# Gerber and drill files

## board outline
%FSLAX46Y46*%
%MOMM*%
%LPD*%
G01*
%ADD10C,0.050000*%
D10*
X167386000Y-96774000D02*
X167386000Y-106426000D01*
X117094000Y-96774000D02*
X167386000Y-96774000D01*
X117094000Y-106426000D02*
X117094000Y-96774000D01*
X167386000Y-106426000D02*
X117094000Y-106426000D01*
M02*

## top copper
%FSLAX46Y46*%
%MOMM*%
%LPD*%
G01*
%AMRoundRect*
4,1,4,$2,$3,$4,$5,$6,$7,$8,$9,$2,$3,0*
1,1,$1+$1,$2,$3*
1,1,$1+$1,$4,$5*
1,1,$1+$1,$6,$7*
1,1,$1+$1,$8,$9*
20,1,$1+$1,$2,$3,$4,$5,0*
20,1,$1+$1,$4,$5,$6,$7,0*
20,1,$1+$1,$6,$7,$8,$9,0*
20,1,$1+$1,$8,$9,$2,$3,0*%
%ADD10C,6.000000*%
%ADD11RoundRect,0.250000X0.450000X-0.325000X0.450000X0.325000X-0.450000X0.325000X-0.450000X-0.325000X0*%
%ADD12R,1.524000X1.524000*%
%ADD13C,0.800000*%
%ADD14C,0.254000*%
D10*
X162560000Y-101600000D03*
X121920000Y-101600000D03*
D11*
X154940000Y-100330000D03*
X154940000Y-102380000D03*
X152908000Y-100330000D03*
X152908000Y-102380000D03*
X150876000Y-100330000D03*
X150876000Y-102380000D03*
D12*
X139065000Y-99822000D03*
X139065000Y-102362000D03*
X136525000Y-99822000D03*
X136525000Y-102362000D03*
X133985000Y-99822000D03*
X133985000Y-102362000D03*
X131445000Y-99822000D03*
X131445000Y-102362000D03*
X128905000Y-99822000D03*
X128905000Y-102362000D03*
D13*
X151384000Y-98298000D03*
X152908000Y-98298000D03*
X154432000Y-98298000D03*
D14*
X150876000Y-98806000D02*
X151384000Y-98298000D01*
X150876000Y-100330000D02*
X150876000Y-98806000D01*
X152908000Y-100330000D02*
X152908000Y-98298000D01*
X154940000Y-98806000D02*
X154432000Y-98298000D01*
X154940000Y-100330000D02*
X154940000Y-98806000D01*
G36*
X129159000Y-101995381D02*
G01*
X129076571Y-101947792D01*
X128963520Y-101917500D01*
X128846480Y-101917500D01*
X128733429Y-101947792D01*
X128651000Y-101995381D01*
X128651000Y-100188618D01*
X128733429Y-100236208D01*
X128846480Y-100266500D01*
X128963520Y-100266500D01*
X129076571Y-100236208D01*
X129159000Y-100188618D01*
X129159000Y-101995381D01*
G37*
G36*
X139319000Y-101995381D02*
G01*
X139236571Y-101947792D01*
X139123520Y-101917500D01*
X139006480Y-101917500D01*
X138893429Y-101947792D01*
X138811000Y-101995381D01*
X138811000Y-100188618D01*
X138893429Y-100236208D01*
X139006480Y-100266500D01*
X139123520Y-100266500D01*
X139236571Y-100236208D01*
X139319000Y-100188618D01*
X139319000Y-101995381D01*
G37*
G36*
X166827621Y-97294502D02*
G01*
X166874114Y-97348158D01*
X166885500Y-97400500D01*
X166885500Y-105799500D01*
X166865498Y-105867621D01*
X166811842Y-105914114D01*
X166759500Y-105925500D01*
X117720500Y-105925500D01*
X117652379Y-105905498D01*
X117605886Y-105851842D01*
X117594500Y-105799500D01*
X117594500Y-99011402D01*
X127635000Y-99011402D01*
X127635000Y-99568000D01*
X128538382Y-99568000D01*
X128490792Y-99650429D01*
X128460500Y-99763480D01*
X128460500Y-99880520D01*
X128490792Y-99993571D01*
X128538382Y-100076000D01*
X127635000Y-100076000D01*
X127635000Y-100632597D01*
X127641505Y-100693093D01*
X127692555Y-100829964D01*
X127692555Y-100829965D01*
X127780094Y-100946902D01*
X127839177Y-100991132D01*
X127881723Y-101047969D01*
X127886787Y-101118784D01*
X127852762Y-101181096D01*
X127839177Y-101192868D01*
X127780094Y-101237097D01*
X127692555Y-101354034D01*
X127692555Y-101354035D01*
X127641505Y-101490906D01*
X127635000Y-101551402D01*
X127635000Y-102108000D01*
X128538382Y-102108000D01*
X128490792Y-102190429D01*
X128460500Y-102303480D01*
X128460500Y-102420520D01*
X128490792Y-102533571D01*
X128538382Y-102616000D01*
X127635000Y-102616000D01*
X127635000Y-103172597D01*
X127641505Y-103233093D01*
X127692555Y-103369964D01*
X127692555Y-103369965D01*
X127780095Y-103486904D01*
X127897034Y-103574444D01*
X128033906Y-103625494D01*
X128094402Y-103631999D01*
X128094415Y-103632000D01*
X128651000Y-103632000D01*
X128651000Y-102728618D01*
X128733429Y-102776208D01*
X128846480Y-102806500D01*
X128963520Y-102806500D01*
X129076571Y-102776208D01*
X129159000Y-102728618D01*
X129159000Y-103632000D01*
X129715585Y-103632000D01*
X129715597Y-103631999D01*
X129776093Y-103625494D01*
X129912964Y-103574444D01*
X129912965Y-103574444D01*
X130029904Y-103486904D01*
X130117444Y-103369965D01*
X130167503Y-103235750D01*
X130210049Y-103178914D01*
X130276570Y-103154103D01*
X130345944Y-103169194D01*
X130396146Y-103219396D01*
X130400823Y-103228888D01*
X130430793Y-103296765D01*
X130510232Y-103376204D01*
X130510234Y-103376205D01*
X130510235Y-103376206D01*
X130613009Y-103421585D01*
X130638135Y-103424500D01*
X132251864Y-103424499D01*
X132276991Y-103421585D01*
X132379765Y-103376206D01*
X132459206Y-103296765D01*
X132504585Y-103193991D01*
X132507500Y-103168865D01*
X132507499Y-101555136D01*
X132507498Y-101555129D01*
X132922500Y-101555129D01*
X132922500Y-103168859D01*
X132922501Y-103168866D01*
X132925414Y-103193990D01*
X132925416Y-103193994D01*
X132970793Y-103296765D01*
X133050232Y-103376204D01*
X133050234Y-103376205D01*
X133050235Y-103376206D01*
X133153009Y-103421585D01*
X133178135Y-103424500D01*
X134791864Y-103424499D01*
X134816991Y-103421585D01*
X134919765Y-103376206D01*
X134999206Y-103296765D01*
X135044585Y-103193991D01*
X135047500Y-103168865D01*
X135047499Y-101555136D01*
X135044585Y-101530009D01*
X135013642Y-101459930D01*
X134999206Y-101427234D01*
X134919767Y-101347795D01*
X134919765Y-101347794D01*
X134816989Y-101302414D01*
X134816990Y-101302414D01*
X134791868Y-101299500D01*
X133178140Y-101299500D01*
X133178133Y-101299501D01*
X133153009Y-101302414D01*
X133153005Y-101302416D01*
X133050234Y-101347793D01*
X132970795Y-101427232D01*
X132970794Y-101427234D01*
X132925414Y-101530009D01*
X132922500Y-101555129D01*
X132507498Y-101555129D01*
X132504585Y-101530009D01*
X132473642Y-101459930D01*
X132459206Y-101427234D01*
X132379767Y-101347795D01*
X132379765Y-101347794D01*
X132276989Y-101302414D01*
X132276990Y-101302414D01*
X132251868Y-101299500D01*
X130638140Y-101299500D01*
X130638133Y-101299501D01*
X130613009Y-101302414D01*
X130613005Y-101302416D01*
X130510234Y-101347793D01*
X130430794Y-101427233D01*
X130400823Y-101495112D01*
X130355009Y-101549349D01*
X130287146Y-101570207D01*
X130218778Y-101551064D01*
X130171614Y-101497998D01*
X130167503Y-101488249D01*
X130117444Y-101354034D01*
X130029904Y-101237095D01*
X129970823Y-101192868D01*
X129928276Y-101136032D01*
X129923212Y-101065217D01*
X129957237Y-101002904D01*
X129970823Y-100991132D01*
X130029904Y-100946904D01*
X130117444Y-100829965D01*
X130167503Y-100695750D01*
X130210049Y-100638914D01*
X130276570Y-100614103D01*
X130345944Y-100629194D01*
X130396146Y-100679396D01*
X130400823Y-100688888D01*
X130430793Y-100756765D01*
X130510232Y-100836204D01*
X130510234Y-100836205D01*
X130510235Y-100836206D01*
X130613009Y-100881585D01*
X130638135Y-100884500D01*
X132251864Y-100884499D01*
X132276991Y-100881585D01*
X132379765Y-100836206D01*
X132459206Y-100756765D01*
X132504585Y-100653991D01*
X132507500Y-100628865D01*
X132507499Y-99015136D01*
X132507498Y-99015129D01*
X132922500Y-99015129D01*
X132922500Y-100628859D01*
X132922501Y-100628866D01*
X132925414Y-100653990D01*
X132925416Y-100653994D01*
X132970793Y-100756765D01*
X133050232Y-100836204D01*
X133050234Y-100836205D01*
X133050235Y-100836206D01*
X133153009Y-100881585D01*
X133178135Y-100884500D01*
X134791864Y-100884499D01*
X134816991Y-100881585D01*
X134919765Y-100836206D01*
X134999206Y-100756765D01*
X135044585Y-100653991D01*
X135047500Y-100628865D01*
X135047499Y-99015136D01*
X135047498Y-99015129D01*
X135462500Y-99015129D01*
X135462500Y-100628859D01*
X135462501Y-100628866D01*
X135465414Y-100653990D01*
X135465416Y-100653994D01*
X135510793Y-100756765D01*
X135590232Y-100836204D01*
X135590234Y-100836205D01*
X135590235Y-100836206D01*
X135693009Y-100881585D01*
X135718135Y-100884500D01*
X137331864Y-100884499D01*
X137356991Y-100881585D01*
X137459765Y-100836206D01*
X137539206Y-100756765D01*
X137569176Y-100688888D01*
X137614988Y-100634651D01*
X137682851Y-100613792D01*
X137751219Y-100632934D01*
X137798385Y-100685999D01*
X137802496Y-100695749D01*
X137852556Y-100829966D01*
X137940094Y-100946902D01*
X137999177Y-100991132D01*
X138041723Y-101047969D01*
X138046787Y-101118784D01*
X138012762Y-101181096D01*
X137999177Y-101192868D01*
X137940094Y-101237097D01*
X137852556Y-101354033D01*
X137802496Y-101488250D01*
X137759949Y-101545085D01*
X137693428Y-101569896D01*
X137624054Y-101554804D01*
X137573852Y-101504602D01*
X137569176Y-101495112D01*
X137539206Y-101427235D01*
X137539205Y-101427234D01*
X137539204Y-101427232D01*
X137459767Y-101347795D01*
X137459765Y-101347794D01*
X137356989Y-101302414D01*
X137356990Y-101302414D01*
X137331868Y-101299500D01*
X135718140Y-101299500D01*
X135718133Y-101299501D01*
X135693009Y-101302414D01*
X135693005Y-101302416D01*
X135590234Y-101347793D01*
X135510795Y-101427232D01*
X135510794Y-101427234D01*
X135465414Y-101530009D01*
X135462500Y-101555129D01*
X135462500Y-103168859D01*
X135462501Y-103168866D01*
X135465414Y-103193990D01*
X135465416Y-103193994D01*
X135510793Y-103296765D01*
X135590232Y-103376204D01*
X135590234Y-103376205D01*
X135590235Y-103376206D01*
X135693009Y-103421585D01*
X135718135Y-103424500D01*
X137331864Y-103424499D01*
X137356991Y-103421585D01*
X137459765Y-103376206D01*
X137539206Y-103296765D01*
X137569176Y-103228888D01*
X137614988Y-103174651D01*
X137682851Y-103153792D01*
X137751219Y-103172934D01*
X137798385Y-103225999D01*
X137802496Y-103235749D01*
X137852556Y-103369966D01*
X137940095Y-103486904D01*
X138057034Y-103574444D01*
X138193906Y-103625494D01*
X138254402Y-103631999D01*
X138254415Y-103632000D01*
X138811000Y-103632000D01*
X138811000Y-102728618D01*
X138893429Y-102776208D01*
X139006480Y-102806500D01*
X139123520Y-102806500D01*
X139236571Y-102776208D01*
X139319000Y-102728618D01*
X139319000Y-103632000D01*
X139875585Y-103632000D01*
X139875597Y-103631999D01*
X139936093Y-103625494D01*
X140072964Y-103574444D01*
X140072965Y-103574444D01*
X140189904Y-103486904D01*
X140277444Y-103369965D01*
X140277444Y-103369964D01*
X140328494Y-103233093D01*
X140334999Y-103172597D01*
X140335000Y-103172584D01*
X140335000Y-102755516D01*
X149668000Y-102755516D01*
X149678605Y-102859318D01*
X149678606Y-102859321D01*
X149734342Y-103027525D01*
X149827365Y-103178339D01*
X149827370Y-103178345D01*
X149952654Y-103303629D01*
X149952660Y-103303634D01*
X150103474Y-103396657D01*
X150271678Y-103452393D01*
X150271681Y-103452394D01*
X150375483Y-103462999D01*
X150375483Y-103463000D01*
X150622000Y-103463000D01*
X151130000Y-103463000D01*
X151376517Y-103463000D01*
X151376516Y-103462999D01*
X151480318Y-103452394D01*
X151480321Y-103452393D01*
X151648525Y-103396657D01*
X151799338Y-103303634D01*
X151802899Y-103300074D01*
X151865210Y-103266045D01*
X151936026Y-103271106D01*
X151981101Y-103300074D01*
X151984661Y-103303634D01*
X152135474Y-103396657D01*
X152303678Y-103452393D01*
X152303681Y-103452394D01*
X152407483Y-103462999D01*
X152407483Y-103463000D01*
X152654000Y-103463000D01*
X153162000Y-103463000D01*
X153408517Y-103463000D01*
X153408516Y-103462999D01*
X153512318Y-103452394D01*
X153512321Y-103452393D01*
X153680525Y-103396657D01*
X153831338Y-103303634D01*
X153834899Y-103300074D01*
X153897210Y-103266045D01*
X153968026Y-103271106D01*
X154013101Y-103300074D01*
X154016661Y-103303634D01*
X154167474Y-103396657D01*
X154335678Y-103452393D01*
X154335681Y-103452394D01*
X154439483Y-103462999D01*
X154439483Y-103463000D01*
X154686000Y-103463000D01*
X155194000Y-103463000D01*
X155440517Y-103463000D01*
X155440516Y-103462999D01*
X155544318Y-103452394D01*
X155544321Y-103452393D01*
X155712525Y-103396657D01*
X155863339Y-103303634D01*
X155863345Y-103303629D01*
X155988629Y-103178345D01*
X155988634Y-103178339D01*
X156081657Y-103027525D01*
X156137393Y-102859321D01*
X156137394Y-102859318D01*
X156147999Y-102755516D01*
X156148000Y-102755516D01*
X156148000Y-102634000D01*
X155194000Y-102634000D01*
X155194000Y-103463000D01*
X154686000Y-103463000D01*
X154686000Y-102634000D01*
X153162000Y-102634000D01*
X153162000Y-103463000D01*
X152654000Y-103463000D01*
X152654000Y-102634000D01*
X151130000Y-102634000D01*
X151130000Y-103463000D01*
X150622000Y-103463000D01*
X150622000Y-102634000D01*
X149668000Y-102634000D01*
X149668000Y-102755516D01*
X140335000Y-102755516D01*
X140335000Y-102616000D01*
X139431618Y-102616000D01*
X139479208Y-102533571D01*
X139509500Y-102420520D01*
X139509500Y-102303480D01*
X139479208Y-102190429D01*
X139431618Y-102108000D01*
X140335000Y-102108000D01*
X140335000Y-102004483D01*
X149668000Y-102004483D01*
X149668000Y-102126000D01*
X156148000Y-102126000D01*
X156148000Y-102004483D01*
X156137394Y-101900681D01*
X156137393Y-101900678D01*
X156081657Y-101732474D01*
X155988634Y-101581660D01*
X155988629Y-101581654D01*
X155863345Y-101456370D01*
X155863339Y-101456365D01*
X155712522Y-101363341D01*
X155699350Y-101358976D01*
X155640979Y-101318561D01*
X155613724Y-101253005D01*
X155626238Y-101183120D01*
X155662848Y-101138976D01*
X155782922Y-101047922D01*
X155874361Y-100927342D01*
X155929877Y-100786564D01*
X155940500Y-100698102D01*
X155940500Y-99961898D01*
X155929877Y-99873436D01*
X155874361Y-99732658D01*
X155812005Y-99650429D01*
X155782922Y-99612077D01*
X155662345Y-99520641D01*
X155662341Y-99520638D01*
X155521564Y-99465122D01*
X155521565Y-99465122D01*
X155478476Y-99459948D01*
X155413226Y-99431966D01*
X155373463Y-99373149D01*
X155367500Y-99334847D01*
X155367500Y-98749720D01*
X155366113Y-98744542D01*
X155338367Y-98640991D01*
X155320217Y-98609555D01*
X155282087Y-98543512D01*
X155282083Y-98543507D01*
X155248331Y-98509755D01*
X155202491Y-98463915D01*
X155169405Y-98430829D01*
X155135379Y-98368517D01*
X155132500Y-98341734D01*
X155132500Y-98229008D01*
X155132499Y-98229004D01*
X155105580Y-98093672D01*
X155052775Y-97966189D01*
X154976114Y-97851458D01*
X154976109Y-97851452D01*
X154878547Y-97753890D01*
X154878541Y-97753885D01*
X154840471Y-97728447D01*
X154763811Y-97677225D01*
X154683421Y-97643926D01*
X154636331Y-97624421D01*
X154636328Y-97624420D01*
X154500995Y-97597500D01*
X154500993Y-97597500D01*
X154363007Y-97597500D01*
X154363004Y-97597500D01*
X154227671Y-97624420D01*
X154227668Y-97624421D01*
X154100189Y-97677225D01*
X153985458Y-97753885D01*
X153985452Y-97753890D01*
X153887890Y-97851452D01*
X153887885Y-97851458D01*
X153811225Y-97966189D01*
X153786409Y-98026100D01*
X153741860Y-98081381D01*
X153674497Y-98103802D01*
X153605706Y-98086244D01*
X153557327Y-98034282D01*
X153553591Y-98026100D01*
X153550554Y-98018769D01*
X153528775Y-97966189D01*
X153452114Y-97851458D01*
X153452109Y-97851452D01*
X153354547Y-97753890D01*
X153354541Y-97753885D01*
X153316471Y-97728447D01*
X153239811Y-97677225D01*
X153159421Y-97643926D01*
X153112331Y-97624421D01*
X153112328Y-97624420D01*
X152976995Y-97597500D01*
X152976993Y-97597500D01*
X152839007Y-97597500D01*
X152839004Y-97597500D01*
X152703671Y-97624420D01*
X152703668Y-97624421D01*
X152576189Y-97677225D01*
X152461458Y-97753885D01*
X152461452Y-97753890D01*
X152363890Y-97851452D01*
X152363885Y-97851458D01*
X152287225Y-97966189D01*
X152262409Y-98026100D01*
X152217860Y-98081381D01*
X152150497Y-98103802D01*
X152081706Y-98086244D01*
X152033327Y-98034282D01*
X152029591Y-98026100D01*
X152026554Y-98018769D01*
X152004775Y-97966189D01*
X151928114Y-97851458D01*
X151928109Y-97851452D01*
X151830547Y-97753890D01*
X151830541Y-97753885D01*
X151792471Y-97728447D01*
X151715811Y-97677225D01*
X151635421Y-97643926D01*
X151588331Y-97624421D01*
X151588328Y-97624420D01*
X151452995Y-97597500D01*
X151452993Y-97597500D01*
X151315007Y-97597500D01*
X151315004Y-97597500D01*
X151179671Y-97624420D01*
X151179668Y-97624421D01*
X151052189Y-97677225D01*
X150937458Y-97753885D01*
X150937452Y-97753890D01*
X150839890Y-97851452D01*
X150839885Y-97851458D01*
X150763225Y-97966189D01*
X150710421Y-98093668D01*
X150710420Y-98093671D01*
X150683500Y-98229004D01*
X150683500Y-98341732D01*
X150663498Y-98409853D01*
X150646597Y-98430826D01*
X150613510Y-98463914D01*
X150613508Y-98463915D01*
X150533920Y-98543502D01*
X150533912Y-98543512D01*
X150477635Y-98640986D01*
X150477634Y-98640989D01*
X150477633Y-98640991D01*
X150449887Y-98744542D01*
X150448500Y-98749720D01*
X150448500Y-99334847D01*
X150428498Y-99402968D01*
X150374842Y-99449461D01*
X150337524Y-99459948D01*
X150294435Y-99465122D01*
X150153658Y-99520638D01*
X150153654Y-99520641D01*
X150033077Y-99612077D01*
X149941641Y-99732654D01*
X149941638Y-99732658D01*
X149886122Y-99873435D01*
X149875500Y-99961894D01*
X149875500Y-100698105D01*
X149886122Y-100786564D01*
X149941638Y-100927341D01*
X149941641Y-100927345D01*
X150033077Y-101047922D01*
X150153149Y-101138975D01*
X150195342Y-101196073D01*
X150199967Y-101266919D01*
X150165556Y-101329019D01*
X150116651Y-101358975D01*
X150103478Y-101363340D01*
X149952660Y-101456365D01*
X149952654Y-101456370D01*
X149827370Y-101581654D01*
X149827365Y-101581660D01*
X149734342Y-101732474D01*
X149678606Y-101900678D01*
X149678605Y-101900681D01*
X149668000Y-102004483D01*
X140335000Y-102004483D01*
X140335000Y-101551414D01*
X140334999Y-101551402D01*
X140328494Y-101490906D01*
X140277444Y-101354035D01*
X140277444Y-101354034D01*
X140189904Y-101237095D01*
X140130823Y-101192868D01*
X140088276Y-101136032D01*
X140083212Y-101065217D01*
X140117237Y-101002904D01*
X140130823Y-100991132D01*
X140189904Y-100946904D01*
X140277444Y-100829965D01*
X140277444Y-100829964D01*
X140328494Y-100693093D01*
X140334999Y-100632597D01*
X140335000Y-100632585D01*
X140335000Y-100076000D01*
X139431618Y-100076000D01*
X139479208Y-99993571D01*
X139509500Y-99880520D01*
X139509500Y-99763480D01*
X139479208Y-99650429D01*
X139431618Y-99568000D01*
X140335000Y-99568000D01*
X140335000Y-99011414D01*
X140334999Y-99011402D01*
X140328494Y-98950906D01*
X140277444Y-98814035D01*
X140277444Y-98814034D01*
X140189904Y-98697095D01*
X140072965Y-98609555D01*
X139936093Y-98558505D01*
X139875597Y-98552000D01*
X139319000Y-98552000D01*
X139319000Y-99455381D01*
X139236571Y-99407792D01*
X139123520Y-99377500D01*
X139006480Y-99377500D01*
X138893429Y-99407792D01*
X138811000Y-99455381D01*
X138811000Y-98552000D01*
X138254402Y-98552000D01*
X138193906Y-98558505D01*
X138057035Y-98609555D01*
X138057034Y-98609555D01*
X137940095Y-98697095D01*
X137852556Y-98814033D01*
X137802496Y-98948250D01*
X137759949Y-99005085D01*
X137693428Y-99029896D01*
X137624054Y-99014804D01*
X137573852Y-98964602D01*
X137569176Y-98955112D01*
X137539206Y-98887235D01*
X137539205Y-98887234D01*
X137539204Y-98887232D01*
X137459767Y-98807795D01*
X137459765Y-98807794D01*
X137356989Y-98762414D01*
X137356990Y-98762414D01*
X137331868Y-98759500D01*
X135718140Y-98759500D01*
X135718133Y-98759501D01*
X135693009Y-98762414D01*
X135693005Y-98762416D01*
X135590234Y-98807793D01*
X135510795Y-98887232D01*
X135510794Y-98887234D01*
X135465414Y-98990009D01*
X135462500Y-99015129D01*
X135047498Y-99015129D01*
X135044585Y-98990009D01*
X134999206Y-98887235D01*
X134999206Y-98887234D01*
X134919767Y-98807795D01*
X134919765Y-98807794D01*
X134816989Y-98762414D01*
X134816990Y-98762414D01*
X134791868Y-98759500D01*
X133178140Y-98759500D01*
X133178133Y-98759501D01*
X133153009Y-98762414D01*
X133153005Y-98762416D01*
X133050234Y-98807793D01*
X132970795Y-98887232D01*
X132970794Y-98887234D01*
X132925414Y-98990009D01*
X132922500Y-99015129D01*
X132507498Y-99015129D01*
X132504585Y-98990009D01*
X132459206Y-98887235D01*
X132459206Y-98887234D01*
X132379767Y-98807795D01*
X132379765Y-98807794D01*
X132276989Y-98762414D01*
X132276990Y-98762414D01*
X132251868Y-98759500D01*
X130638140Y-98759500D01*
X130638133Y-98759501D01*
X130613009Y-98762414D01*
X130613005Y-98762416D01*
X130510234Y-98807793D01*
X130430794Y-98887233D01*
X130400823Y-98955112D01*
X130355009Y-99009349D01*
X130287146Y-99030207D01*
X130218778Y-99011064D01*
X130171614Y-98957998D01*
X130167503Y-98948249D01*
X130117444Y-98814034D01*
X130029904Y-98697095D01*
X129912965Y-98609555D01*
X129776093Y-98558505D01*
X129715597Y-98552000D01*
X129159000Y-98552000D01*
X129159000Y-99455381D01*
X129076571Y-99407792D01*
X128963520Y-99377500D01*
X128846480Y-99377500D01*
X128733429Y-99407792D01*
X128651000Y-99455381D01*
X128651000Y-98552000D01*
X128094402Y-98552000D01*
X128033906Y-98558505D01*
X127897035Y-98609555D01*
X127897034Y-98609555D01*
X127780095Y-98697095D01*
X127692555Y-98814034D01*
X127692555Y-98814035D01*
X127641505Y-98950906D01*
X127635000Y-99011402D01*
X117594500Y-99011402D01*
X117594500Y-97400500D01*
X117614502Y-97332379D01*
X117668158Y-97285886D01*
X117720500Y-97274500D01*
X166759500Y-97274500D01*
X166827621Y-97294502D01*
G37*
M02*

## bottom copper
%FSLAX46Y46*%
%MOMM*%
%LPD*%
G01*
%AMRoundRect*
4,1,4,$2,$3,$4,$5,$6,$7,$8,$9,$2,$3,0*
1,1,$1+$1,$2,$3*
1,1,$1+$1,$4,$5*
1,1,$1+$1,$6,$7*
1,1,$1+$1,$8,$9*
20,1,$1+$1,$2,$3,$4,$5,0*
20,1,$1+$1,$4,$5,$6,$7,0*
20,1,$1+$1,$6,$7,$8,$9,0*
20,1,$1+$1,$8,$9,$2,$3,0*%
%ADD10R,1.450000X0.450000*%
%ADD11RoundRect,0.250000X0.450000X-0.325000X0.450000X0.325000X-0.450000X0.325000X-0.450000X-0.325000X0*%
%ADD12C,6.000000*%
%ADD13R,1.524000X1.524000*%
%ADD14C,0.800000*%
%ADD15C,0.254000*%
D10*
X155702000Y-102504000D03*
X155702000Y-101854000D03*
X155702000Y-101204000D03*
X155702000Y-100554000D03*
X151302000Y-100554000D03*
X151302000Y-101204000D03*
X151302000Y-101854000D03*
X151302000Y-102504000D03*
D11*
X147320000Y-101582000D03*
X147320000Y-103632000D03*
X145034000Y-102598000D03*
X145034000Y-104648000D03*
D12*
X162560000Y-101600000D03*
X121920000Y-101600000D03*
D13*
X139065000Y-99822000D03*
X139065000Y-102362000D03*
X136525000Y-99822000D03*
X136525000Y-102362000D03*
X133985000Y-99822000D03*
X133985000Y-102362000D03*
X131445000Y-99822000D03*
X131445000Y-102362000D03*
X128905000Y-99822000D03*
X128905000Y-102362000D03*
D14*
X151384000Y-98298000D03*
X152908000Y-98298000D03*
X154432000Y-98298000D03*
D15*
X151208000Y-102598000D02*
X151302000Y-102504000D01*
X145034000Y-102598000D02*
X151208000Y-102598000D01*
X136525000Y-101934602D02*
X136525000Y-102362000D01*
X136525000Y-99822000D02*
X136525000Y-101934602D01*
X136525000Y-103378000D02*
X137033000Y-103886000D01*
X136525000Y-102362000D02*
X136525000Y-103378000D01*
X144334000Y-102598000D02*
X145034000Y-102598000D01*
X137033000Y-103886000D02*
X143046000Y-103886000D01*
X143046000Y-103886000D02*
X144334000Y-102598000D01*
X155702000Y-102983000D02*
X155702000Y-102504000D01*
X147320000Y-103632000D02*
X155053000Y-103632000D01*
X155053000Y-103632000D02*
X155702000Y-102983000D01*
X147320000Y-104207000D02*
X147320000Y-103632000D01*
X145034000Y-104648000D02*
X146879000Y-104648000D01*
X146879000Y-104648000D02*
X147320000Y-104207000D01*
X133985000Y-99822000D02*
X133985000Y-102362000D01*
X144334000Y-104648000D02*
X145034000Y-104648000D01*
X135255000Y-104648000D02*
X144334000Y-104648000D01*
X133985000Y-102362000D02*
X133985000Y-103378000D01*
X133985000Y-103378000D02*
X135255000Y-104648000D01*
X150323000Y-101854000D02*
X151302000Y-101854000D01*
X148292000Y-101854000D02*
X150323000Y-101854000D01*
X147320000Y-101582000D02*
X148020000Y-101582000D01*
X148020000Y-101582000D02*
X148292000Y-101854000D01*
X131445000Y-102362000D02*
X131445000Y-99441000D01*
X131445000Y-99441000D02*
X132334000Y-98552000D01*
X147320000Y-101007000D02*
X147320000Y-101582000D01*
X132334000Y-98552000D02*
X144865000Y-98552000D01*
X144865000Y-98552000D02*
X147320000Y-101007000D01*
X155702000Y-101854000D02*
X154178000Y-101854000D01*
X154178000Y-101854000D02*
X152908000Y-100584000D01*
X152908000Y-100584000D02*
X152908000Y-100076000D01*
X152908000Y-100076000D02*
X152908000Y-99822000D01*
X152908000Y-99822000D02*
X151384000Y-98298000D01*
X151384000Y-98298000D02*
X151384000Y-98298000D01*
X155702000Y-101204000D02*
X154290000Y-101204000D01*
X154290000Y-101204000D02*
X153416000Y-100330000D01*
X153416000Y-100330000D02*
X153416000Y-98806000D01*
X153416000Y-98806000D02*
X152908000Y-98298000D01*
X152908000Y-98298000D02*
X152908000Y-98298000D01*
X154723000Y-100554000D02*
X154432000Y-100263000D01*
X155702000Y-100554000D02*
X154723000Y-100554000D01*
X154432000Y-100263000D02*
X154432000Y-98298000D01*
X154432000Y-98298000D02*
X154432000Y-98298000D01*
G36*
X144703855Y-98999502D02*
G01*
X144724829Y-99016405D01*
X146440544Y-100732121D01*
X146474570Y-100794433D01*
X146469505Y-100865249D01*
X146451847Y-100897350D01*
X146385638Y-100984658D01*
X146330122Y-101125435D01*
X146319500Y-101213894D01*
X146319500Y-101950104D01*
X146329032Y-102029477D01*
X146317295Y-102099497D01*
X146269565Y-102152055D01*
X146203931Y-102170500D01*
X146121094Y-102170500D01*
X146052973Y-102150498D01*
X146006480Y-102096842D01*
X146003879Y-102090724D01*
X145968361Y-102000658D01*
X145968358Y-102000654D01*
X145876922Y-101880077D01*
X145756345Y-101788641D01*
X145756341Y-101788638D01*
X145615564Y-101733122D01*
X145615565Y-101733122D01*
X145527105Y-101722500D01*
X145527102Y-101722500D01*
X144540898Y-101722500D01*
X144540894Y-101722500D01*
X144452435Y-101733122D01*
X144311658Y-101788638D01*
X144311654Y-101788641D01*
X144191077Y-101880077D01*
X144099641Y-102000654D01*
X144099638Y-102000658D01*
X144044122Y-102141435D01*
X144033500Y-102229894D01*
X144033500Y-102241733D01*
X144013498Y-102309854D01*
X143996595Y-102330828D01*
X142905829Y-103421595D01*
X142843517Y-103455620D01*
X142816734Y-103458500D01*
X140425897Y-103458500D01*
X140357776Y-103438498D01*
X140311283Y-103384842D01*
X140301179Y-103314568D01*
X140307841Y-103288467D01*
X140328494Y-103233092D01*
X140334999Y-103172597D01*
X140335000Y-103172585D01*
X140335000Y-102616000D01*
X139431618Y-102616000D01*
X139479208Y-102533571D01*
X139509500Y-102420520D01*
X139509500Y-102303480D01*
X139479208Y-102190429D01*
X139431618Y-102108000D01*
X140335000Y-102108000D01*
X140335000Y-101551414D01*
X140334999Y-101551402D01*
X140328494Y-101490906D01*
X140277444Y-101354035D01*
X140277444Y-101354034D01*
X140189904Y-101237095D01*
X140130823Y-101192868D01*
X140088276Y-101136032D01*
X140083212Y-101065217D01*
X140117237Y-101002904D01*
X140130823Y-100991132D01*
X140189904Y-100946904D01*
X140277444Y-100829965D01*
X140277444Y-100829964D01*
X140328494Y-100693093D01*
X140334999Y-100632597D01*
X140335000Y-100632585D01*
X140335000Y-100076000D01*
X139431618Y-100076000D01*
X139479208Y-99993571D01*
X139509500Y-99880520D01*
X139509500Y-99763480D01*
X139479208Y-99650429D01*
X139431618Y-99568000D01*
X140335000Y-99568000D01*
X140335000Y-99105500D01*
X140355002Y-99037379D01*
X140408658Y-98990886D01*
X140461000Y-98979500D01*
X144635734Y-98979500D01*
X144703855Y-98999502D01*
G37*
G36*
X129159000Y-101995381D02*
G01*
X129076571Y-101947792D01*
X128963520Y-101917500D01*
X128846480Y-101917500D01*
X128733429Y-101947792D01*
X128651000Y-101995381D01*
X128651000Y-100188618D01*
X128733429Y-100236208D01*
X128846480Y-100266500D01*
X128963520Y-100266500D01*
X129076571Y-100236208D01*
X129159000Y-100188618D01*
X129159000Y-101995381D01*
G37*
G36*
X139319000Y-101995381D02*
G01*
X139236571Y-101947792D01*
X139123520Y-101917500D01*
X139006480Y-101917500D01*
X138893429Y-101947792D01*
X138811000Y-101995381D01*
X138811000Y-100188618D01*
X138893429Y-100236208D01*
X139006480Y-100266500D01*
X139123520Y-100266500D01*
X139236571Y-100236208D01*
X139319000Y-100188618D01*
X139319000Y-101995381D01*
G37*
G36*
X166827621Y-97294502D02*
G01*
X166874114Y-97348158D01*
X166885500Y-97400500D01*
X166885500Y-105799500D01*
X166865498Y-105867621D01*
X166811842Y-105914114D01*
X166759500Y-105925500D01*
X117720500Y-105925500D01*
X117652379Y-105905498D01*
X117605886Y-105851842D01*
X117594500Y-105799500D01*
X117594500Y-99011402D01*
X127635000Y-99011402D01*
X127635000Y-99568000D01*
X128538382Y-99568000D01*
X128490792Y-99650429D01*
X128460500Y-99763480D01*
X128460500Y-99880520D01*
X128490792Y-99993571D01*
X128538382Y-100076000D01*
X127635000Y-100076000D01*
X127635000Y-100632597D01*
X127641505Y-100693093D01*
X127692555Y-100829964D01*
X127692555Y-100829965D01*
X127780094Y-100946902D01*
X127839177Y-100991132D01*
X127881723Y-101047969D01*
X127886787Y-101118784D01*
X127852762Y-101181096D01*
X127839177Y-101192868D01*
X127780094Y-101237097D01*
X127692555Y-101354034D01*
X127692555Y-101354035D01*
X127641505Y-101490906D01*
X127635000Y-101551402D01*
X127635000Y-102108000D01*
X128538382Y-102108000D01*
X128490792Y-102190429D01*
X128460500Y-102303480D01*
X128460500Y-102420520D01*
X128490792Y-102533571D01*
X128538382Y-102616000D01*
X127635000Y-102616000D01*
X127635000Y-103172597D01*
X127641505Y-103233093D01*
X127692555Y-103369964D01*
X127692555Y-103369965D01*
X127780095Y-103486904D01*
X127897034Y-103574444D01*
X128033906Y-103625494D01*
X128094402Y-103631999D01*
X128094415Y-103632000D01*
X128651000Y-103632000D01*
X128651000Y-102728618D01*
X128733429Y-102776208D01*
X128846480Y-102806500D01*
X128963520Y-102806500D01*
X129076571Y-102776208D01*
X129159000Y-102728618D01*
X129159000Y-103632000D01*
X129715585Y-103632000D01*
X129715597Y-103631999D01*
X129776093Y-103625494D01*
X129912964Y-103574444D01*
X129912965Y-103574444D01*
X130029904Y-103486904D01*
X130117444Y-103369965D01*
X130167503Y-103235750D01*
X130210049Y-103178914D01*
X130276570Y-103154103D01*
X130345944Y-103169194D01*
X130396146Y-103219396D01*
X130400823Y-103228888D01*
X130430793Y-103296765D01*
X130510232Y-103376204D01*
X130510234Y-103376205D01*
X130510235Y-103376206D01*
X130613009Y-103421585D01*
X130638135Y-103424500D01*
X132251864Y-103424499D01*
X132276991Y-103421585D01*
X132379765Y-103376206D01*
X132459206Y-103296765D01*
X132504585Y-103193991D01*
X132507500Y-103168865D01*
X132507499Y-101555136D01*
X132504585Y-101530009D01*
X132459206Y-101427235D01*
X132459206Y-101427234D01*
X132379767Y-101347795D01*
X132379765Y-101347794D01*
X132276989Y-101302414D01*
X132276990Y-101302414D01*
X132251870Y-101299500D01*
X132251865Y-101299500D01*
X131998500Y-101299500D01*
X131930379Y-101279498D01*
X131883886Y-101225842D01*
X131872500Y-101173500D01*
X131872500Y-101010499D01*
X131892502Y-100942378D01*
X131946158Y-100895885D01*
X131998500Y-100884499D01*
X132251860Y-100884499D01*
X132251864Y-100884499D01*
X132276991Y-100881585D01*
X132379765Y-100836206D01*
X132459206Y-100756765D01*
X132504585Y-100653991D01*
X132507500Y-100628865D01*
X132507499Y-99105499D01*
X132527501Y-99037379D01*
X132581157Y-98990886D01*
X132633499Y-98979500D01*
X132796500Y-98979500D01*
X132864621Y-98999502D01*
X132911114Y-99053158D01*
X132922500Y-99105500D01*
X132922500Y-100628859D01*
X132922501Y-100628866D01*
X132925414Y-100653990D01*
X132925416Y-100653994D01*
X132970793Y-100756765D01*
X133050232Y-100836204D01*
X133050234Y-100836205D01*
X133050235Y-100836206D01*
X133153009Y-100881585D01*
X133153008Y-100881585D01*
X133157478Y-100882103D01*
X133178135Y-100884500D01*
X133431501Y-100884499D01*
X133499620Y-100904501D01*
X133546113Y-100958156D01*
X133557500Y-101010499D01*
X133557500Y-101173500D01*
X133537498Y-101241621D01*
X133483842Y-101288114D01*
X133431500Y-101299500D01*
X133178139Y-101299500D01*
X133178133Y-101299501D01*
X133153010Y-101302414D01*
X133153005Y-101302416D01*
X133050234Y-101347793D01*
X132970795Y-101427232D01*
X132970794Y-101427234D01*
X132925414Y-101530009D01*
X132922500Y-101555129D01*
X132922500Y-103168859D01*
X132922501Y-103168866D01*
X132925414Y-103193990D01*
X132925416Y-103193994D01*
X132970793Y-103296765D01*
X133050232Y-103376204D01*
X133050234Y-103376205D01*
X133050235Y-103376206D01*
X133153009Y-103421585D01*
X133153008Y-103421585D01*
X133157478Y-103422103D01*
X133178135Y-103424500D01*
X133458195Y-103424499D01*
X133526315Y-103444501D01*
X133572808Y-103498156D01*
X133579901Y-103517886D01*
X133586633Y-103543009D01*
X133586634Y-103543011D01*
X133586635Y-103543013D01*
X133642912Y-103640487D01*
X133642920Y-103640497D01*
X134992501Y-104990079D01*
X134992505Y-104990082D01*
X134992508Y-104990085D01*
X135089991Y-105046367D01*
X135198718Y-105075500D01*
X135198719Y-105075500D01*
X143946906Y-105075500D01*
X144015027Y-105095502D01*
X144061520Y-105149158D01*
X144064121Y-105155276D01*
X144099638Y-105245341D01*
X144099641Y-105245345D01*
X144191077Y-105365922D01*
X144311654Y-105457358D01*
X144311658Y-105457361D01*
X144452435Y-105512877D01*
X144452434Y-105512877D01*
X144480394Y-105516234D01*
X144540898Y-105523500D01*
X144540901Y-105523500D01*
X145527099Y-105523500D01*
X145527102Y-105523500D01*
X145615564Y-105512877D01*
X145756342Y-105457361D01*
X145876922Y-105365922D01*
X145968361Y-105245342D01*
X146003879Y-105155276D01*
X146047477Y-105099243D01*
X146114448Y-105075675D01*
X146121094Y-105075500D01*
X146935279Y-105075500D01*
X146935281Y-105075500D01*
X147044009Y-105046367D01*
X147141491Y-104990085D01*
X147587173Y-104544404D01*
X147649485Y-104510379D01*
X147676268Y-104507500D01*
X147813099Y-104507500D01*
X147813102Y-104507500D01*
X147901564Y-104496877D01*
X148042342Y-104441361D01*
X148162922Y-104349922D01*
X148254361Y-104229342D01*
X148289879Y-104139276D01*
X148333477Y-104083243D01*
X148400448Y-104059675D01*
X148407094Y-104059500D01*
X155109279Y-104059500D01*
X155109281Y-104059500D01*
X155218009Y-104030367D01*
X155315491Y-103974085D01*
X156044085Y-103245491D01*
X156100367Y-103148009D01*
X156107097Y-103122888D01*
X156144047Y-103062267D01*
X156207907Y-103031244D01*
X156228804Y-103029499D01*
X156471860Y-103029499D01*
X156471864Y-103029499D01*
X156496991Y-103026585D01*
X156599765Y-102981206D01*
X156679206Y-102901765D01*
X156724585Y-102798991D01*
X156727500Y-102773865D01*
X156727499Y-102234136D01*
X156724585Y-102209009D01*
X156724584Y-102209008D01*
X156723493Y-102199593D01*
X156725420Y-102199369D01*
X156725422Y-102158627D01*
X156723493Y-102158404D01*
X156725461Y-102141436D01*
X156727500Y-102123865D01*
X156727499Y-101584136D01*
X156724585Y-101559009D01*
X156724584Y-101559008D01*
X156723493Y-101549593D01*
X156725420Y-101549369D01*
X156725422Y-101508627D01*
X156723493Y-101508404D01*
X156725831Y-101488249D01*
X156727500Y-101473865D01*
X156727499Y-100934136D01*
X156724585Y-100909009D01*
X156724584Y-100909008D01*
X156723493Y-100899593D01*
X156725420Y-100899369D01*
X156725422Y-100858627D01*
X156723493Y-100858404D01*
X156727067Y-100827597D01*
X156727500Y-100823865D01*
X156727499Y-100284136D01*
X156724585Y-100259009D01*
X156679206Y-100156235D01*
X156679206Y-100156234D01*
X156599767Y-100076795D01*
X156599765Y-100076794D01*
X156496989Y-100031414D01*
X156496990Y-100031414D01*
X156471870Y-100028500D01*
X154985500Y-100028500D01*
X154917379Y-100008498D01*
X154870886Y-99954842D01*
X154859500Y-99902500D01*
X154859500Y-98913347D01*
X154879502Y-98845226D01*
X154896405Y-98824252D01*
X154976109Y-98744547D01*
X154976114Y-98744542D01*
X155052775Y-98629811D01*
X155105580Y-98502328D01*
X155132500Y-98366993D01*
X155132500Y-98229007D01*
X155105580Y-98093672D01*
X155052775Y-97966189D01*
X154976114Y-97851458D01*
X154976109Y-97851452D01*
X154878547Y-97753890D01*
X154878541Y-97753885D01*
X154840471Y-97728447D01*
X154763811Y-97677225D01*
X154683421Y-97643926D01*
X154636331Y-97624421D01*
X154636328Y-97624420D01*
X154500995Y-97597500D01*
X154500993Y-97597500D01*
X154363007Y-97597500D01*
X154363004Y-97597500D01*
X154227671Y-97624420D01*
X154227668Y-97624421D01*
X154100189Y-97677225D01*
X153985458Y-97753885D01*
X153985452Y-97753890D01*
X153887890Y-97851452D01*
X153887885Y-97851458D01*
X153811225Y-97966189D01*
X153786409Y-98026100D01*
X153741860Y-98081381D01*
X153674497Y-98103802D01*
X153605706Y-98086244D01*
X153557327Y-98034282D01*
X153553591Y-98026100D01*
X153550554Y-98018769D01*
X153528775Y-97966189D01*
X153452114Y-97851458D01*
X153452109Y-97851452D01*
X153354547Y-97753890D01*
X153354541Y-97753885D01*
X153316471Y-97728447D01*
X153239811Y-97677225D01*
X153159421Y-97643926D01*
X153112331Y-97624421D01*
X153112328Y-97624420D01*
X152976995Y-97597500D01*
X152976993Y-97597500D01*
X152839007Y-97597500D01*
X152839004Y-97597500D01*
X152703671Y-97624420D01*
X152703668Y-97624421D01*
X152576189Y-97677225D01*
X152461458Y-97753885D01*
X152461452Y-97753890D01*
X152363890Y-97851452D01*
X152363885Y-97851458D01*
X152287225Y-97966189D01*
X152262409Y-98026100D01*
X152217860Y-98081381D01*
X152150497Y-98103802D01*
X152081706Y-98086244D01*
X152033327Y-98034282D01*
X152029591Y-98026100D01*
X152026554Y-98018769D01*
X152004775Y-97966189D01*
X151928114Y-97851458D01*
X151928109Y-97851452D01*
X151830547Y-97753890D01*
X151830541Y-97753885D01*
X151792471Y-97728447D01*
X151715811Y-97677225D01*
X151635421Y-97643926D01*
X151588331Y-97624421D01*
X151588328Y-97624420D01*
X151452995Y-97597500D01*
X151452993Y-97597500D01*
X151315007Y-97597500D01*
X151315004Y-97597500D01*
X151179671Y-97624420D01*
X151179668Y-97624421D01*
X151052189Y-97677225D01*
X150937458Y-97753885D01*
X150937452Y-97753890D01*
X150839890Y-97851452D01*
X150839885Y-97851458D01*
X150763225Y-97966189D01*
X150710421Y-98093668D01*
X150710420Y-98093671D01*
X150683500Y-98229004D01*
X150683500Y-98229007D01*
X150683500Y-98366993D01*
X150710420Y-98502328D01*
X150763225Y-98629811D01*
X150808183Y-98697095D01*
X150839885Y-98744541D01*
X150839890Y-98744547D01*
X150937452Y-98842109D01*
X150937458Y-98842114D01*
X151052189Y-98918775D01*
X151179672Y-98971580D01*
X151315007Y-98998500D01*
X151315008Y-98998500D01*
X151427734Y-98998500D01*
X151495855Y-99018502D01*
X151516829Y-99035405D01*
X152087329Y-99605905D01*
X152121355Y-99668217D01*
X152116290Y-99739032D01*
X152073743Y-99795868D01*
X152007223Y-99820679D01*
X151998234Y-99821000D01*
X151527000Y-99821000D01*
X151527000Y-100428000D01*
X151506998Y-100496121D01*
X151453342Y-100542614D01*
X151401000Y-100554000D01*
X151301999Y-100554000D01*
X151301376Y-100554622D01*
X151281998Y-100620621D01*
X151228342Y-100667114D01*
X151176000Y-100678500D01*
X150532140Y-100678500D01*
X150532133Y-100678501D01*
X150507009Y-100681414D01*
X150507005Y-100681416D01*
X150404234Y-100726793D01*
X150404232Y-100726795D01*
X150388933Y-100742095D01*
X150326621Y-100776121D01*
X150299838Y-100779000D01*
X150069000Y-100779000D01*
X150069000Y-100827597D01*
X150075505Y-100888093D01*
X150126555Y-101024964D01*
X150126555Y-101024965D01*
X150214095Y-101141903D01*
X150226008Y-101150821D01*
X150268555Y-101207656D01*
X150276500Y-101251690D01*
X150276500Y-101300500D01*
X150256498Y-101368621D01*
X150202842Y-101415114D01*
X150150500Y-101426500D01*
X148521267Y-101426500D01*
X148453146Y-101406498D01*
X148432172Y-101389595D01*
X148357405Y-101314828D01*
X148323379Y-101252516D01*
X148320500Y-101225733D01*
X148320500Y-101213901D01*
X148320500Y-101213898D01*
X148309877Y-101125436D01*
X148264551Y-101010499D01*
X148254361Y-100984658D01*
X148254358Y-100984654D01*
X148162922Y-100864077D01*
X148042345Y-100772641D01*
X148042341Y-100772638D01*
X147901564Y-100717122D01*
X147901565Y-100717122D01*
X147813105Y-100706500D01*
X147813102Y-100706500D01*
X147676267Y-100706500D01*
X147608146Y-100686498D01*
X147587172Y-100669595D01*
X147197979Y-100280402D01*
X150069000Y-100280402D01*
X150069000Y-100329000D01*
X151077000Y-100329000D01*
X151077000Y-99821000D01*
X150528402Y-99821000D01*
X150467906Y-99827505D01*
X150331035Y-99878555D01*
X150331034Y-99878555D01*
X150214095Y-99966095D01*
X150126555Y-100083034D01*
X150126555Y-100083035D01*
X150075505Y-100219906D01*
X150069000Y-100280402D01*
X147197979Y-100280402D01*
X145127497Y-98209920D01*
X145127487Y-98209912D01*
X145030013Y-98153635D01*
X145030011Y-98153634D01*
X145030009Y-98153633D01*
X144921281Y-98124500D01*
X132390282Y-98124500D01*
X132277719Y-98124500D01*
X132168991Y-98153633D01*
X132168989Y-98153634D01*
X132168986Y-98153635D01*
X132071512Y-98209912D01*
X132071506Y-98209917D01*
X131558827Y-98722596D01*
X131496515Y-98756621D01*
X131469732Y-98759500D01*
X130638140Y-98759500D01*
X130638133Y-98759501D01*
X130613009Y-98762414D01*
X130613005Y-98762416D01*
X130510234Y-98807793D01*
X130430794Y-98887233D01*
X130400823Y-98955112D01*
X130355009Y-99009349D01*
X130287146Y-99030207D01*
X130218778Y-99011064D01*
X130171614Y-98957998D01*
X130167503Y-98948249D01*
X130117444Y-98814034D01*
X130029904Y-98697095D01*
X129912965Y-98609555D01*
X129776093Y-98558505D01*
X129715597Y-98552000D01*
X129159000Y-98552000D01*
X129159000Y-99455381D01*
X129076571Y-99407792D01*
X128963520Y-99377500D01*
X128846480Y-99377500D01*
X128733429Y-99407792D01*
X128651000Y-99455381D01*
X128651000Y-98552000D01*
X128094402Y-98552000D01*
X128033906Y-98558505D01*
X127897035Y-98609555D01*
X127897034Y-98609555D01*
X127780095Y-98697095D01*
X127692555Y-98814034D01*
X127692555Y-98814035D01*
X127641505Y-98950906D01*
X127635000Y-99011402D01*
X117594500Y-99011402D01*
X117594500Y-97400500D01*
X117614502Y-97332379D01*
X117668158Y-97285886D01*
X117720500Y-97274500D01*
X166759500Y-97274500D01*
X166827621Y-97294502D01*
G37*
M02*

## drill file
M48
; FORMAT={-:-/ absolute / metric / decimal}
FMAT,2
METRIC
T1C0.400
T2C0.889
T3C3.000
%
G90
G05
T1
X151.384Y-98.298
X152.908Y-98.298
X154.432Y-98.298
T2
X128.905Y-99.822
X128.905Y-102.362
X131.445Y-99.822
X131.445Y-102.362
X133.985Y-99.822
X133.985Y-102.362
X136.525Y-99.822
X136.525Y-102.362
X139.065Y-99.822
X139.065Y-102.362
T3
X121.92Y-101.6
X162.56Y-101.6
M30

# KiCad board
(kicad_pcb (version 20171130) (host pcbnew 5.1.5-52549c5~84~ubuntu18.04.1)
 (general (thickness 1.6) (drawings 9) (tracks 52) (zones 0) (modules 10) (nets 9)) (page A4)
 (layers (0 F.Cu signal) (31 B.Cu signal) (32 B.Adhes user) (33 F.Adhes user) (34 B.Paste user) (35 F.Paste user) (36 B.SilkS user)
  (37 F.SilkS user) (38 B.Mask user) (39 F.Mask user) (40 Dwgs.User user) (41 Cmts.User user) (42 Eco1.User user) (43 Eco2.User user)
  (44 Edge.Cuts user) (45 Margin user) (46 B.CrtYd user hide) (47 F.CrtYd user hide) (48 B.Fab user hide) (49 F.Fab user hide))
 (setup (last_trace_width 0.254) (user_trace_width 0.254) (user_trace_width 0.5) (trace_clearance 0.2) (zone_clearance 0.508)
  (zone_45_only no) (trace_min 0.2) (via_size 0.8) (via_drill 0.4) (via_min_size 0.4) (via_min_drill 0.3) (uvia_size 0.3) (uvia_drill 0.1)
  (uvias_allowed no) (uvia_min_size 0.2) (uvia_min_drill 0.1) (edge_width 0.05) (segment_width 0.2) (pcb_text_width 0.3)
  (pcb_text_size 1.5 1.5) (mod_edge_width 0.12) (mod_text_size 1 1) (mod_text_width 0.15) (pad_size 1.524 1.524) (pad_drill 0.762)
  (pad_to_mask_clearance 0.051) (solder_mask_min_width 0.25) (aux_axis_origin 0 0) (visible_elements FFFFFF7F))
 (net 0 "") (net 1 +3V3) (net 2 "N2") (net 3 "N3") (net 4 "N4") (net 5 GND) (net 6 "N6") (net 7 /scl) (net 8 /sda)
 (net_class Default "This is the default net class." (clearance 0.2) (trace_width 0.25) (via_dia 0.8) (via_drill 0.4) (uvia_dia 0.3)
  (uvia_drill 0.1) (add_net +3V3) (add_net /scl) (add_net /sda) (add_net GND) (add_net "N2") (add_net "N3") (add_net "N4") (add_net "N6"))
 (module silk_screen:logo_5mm (layer F.Cu) (at 145.288 101.346 90)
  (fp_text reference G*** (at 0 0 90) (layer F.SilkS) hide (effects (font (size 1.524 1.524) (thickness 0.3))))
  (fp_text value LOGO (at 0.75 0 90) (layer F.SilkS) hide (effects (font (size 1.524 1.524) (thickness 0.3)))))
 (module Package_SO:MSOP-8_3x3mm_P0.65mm (layer B.Cu) (at 153.502 101.529)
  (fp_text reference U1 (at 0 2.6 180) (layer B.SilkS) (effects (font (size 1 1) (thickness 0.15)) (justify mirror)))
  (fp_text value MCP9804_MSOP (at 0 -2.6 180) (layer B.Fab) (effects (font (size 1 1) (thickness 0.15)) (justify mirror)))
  (pad 8 smd rect (at 2.2 0.975) (size 1.45 0.45) (layers B.Cu B.Paste B.Mask) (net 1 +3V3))
  (pad 7 smd rect (at 2.2 0.325) (size 1.45 0.45) (layers B.Cu B.Paste B.Mask) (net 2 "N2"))
  (pad 6 smd rect (at 2.2 -0.325) (size 1.45 0.45) (layers B.Cu B.Paste B.Mask) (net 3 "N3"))
  (pad 5 smd rect (at 2.2 -0.975) (size 1.45 0.45) (layers B.Cu B.Paste B.Mask) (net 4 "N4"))
  (pad 4 smd rect (at -2.2 -0.975) (size 1.45 0.45) (layers B.Cu B.Paste B.Mask) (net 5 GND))
  (pad 3 smd rect (at -2.2 -0.325) (size 1.45 0.45) (layers B.Cu B.Paste B.Mask) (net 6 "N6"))
  (pad 2 smd rect (at -2.2 0.325) (size 1.45 0.45) (layers B.Cu B.Paste B.Mask) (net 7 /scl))
  (pad 1 smd rect (at -2.2 0.975) (size 1.45 0.45) (layers B.Cu B.Paste B.Mask) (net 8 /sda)))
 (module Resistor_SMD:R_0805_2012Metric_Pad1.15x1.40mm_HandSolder (layer B.Cu) (at 147.32 102.607 90)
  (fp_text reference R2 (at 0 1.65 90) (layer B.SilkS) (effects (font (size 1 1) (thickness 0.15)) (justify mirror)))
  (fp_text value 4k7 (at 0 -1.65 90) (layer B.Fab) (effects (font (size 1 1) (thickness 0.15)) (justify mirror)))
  (pad 2 smd roundrect (at 1.025 0 90) (size 1.15 1.4) (layers B.Cu B.Paste B.Mask) (roundrect_rratio 0.217391) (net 7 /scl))
  (pad 1 smd roundrect (at -1.025 0 90) (size 1.15 1.4) (layers B.Cu B.Paste B.Mask) (roundrect_rratio 0.217391) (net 1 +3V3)))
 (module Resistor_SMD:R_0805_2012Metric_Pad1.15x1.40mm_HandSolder (layer B.Cu) (at 145.034 103.623 90)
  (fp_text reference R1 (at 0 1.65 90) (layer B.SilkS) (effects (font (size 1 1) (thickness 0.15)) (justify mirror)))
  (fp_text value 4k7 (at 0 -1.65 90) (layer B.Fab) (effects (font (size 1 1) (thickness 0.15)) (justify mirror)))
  (pad 2 smd roundrect (at 1.025 0 90) (size 1.15 1.4) (layers B.Cu B.Paste B.Mask) (roundrect_rratio 0.217391) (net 8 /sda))
  (pad 1 smd roundrect (at -1.025 0 90) (size 1.15 1.4) (layers B.Cu B.Paste B.Mask) (roundrect_rratio 0.217391) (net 1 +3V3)))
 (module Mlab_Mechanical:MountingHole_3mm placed (layer F.Cu) (at 162.56 101.6)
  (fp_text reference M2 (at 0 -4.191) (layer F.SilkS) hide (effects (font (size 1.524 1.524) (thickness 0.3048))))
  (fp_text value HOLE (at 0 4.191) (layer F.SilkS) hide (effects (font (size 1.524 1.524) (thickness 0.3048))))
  (pad 1 thru_hole circle (at 0 0) (size 6 6) (drill 3) (layers *.Cu *.Adhes *.Mask) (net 5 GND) (clearance 1) (zone_connect 2)))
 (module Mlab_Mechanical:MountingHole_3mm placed (layer F.Cu) (at 121.92 101.6)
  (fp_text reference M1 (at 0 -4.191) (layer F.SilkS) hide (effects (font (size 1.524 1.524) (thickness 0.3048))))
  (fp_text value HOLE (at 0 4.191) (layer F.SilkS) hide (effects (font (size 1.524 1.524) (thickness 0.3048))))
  (pad 1 thru_hole circle (at 0 0) (size 6 6) (drill 3) (layers *.Cu *.Adhes *.Mask) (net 5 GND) (clearance 1) (zone_connect 2)))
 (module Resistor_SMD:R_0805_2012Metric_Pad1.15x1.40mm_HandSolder (layer F.Cu) (at 154.94 101.355 90)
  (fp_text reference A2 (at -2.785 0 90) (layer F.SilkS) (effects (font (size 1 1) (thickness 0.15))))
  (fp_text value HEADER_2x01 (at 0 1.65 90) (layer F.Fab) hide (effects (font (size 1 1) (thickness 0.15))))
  (pad 2 smd roundrect (at 1.025 0 90) (size 1.15 1.4) (layers F.Cu F.Paste F.Mask) (roundrect_rratio 0.217391) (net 4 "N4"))
  (pad 1 smd roundrect (at -1.025 0 90) (size 1.15 1.4) (layers F.Cu F.Paste F.Mask) (roundrect_rratio 0.217391) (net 5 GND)))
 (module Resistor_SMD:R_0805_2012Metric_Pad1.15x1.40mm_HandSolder (layer F.Cu) (at 152.908 101.355 90)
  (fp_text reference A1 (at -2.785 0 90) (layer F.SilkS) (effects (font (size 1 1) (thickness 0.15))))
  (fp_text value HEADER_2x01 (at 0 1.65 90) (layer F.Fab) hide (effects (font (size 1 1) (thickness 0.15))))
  (pad 2 smd roundrect (at 1.025 0 90) (size 1.15 1.4) (layers F.Cu F.Paste F.Mask) (roundrect_rratio 0.217391) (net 3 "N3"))
  (pad 1 smd roundrect (at -1.025 0 90) (size 1.15 1.4) (layers F.Cu F.Paste F.Mask) (roundrect_rratio 0.217391) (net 5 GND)))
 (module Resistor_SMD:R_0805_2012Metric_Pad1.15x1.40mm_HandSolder (layer F.Cu) (at 150.876 101.355 90)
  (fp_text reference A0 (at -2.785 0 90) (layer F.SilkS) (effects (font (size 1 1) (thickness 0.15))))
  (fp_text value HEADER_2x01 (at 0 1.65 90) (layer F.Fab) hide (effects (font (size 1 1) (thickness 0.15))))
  (pad 2 smd roundrect (at 1.025 0 90) (size 1.15 1.4) (layers F.Cu F.Paste F.Mask) (roundrect_rratio 0.217391) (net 2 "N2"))
  (pad 1 smd roundrect (at -1.025 0 90) (size 1.15 1.4) (layers F.Cu F.Paste F.Mask) (roundrect_rratio 0.217391) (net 5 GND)))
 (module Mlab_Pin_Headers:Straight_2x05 (layer F.Cu) (at 133.985 101.092 90)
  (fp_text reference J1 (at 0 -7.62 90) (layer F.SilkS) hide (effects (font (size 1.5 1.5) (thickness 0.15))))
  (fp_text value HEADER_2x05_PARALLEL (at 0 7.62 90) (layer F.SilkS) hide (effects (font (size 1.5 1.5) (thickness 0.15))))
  (pad 10 thru_hole rect (at 1.27 5.08 90) (size 1.524 1.524) (drill 0.889) (layers *.Cu *.Mask F.SilkS) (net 5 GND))
  (pad 9 thru_hole rect (at -1.27 5.08 90) (size 1.524 1.524) (drill 0.889) (layers *.Cu *.Mask F.SilkS) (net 5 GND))
  (pad 8 thru_hole rect (at 1.27 2.54 90) (size 1.524 1.524) (drill 0.889) (layers *.Cu *.Mask F.SilkS) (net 8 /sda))
  (pad 7 thru_hole rect (at -1.27 2.54 90) (size 1.524 1.524) (drill 0.889) (layers *.Cu *.Mask F.SilkS) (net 8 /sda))
  (pad 6 thru_hole rect (at 1.27 0 90) (size 1.524 1.524) (drill 0.889) (layers *.Cu *.Mask F.SilkS) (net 1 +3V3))
  (pad 5 thru_hole rect (at -1.27 0 90) (size 1.524 1.524) (drill 0.889) (layers *.Cu *.Mask F.SilkS) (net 1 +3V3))
  (pad 4 thru_hole rect (at 1.27 -2.54 90) (size 1.524 1.524) (drill 0.889) (layers *.Cu *.Mask F.SilkS) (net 7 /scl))
  (pad 3 thru_hole rect (at -1.27 -2.54 90) (size 1.524 1.524) (drill 0.889) (layers *.Cu *.Mask F.SilkS) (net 7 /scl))
  (pad 2 thru_hole rect (at 1.27 -5.08 90) (size 1.524 1.524) (drill 0.889) (layers *.Cu *.Mask F.SilkS) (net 5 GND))
  (pad 1 thru_hole rect (at -1.27 -5.08 90) (size 1.524 1.524) (drill 0.889) (layers *.Cu *.Mask F.SilkS) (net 5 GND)))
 (gr_line (start 167.386 96.774) (end 167.386 106.426) (layer Edge.Cuts) (width 0.05))
 (gr_line (start 117.094 96.774) (end 167.386 96.774) (layer Edge.Cuts) (width 0.05))
 (gr_line (start 117.094 106.426) (end 117.094 96.774) (layer Edge.Cuts) (width 0.05))
 (gr_line (start 167.386 106.426) (end 117.094 106.426) (layer Edge.Cuts) (width 0.05))
 (segment (start 151.208 102.598) (end 151.302 102.504) (width 0.254) (layer B.Cu) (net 8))
 (segment (start 145.034 102.598) (end 151.208 102.598) (width 0.254) (layer B.Cu) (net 8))
 (segment (start 136.525 101.934602) (end 136.525 102.362) (width 0.254) (layer B.Cu) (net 8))
 (segment (start 136.525 99.822) (end 136.525 101.934602) (width 0.254) (layer B.Cu) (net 8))
 (segment (start 136.525 103.378) (end 137.033 103.886) (width 0.254) (layer B.Cu) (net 8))
 (segment (start 136.525 102.362) (end 136.525 103.378) (width 0.254) (layer B.Cu) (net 8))
 (segment (start 144.334 102.598) (end 145.034 102.598) (width 0.254) (layer B.Cu) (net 8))
 (segment (start 137.033 103.886) (end 143.046 103.886) (width 0.254) (layer B.Cu) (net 8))
 (segment (start 143.046 103.886) (end 144.334 102.598) (width 0.254) (layer B.Cu) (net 8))
 (segment (start 155.702 102.983) (end 155.702 102.504) (width 0.254) (layer B.Cu) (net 1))
 (segment (start 147.32 103.632) (end 155.053 103.632) (width 0.254) (layer B.Cu) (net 1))
 (segment (start 155.053 103.632) (end 155.702 102.983) (width 0.254) (layer B.Cu) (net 1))
 (segment (start 147.32 104.207) (end 147.32 103.632) (width 0.254) (layer B.Cu) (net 1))
 (segment (start 145.034 104.648) (end 146.879 104.648) (width 0.254) (layer B.Cu) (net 1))
 (segment (start 146.879 104.648) (end 147.32 104.207) (width 0.254) (layer B.Cu) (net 1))
 (segment (start 133.985 99.822) (end 133.985 102.362) (width 0.254) (layer B.Cu) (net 1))
 (segment (start 144.334 104.648) (end 145.034 104.648) (width 0.254) (layer B.Cu) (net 1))
 (segment (start 135.255 104.648) (end 144.334 104.648) (width 0.254) (layer B.Cu) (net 1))
 (segment (start 133.985 102.362) (end 133.985 103.378) (width 0.254) (layer B.Cu) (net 1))
 (segment (start 133.985 103.378) (end 135.255 104.648) (width 0.254) (layer B.Cu) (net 1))
 (segment (start 150.323 101.854) (end 151.302 101.854) (width 0.254) (layer B.Cu) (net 7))
 (segment (start 148.292 101.854) (end 150.323 101.854) (width 0.254) (layer B.Cu) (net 7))
 (segment (start 147.32 101.582) (end 148.02 101.582) (width 0.254) (layer B.Cu) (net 7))
 (segment (start 148.02 101.582) (end 148.292 101.854) (width 0.254) (layer B.Cu) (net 7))
 (segment (start 131.445 102.362) (end 131.445 99.441) (width 0.254) (layer B.Cu) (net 7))
 (segment (start 131.445 99.441) (end 132.334 98.552) (width 0.254) (layer B.Cu) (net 7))
 (segment (start 147.32 101.007) (end 147.32 101.582) (width 0.254) (layer B.Cu) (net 7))
 (segment (start 132.334 98.552) (end 144.865 98.552) (width 0.254) (layer B.Cu) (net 7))
 (segment (start 144.865 98.552) (end 147.32 101.007) (width 0.254) (layer B.Cu) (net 7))
 (segment (start 155.702 101.854) (end 154.178 101.854) (width 0.254) (layer B.Cu) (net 2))
 (segment (start 154.178 101.854) (end 152.908 100.584) (width 0.254) (layer B.Cu) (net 2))
 (segment (start 152.908 100.584) (end 152.908 100.076) (width 0.254) (layer B.Cu) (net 2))
 (segment (start 152.908 100.076) (end 152.908 99.822) (width 0.254) (layer B.Cu) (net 2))
 (segment (start 152.908 99.822) (end 151.384 98.298) (width 0.254) (layer B.Cu) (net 2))
 (segment (start 151.384 98.298) (end 151.384 98.298) (width 0.254) (layer B.Cu) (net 2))
 (via (at 151.384 98.298) (size 0.8) (drill 0.4) (layers F.Cu B.Cu) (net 2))
 (segment (start 150.876 98.806) (end 151.384 98.298) (width 0.254) (layer F.Cu) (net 2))
 (segment (start 150.876 100.33) (end 150.876 98.806) (width 0.254) (layer F.Cu) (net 2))
 (segment (start 155.702 101.204) (end 154.29 101.204) (width 0.254) (layer B.Cu) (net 3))
 (segment (start 154.29 101.204) (end 153.416 100.33) (width 0.254) (layer B.Cu) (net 3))
 (segment (start 153.416 100.33) (end 153.416 98.806) (width 0.254) (layer B.Cu) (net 3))
 (segment (start 153.416 98.806) (end 152.908 98.298) (width 0.254) (layer B.Cu) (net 3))
 (segment (start 152.908 98.298) (end 152.908 98.298) (width 0.254) (layer B.Cu) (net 3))
 (via (at 152.908 98.298) (size 0.8) (drill 0.4) (layers F.Cu B.Cu) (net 3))
 (segment (start 152.908 100.33) (end 152.908 98.298) (width 0.254) (layer F.Cu) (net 3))
 (segment (start 154.723 100.554) (end 154.432 100.263) (width 0.254) (layer B.Cu) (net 4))
 (segment (start 155.702 100.554) (end 154.723 100.554) (width 0.254) (layer B.Cu) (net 4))
 (segment (start 154.432 100.263) (end 154.432 98.298) (width 0.254) (layer B.Cu) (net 4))
 (segment (start 154.432 98.298) (end 154.432 98.298) (width 0.254) (layer B.Cu) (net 4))
 (via (at 154.432 98.298) (size 0.8) (drill 0.4) (layers F.Cu B.Cu) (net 4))
 (segment (start 154.94 98.806) (end 154.432 98.298) (width 0.254) (layer F.Cu) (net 4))
 (segment (start 154.94 100.33) (end 154.94 98.806) (width 0.254) (layer F.Cu) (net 4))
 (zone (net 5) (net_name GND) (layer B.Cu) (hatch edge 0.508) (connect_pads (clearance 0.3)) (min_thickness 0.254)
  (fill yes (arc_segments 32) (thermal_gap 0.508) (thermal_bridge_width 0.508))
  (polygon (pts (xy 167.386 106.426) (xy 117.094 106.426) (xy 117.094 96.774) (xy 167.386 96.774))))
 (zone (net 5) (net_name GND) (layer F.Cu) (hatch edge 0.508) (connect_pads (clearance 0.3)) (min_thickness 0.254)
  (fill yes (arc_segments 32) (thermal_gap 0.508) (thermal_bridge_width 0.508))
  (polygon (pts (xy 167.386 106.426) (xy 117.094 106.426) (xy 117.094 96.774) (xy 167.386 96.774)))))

